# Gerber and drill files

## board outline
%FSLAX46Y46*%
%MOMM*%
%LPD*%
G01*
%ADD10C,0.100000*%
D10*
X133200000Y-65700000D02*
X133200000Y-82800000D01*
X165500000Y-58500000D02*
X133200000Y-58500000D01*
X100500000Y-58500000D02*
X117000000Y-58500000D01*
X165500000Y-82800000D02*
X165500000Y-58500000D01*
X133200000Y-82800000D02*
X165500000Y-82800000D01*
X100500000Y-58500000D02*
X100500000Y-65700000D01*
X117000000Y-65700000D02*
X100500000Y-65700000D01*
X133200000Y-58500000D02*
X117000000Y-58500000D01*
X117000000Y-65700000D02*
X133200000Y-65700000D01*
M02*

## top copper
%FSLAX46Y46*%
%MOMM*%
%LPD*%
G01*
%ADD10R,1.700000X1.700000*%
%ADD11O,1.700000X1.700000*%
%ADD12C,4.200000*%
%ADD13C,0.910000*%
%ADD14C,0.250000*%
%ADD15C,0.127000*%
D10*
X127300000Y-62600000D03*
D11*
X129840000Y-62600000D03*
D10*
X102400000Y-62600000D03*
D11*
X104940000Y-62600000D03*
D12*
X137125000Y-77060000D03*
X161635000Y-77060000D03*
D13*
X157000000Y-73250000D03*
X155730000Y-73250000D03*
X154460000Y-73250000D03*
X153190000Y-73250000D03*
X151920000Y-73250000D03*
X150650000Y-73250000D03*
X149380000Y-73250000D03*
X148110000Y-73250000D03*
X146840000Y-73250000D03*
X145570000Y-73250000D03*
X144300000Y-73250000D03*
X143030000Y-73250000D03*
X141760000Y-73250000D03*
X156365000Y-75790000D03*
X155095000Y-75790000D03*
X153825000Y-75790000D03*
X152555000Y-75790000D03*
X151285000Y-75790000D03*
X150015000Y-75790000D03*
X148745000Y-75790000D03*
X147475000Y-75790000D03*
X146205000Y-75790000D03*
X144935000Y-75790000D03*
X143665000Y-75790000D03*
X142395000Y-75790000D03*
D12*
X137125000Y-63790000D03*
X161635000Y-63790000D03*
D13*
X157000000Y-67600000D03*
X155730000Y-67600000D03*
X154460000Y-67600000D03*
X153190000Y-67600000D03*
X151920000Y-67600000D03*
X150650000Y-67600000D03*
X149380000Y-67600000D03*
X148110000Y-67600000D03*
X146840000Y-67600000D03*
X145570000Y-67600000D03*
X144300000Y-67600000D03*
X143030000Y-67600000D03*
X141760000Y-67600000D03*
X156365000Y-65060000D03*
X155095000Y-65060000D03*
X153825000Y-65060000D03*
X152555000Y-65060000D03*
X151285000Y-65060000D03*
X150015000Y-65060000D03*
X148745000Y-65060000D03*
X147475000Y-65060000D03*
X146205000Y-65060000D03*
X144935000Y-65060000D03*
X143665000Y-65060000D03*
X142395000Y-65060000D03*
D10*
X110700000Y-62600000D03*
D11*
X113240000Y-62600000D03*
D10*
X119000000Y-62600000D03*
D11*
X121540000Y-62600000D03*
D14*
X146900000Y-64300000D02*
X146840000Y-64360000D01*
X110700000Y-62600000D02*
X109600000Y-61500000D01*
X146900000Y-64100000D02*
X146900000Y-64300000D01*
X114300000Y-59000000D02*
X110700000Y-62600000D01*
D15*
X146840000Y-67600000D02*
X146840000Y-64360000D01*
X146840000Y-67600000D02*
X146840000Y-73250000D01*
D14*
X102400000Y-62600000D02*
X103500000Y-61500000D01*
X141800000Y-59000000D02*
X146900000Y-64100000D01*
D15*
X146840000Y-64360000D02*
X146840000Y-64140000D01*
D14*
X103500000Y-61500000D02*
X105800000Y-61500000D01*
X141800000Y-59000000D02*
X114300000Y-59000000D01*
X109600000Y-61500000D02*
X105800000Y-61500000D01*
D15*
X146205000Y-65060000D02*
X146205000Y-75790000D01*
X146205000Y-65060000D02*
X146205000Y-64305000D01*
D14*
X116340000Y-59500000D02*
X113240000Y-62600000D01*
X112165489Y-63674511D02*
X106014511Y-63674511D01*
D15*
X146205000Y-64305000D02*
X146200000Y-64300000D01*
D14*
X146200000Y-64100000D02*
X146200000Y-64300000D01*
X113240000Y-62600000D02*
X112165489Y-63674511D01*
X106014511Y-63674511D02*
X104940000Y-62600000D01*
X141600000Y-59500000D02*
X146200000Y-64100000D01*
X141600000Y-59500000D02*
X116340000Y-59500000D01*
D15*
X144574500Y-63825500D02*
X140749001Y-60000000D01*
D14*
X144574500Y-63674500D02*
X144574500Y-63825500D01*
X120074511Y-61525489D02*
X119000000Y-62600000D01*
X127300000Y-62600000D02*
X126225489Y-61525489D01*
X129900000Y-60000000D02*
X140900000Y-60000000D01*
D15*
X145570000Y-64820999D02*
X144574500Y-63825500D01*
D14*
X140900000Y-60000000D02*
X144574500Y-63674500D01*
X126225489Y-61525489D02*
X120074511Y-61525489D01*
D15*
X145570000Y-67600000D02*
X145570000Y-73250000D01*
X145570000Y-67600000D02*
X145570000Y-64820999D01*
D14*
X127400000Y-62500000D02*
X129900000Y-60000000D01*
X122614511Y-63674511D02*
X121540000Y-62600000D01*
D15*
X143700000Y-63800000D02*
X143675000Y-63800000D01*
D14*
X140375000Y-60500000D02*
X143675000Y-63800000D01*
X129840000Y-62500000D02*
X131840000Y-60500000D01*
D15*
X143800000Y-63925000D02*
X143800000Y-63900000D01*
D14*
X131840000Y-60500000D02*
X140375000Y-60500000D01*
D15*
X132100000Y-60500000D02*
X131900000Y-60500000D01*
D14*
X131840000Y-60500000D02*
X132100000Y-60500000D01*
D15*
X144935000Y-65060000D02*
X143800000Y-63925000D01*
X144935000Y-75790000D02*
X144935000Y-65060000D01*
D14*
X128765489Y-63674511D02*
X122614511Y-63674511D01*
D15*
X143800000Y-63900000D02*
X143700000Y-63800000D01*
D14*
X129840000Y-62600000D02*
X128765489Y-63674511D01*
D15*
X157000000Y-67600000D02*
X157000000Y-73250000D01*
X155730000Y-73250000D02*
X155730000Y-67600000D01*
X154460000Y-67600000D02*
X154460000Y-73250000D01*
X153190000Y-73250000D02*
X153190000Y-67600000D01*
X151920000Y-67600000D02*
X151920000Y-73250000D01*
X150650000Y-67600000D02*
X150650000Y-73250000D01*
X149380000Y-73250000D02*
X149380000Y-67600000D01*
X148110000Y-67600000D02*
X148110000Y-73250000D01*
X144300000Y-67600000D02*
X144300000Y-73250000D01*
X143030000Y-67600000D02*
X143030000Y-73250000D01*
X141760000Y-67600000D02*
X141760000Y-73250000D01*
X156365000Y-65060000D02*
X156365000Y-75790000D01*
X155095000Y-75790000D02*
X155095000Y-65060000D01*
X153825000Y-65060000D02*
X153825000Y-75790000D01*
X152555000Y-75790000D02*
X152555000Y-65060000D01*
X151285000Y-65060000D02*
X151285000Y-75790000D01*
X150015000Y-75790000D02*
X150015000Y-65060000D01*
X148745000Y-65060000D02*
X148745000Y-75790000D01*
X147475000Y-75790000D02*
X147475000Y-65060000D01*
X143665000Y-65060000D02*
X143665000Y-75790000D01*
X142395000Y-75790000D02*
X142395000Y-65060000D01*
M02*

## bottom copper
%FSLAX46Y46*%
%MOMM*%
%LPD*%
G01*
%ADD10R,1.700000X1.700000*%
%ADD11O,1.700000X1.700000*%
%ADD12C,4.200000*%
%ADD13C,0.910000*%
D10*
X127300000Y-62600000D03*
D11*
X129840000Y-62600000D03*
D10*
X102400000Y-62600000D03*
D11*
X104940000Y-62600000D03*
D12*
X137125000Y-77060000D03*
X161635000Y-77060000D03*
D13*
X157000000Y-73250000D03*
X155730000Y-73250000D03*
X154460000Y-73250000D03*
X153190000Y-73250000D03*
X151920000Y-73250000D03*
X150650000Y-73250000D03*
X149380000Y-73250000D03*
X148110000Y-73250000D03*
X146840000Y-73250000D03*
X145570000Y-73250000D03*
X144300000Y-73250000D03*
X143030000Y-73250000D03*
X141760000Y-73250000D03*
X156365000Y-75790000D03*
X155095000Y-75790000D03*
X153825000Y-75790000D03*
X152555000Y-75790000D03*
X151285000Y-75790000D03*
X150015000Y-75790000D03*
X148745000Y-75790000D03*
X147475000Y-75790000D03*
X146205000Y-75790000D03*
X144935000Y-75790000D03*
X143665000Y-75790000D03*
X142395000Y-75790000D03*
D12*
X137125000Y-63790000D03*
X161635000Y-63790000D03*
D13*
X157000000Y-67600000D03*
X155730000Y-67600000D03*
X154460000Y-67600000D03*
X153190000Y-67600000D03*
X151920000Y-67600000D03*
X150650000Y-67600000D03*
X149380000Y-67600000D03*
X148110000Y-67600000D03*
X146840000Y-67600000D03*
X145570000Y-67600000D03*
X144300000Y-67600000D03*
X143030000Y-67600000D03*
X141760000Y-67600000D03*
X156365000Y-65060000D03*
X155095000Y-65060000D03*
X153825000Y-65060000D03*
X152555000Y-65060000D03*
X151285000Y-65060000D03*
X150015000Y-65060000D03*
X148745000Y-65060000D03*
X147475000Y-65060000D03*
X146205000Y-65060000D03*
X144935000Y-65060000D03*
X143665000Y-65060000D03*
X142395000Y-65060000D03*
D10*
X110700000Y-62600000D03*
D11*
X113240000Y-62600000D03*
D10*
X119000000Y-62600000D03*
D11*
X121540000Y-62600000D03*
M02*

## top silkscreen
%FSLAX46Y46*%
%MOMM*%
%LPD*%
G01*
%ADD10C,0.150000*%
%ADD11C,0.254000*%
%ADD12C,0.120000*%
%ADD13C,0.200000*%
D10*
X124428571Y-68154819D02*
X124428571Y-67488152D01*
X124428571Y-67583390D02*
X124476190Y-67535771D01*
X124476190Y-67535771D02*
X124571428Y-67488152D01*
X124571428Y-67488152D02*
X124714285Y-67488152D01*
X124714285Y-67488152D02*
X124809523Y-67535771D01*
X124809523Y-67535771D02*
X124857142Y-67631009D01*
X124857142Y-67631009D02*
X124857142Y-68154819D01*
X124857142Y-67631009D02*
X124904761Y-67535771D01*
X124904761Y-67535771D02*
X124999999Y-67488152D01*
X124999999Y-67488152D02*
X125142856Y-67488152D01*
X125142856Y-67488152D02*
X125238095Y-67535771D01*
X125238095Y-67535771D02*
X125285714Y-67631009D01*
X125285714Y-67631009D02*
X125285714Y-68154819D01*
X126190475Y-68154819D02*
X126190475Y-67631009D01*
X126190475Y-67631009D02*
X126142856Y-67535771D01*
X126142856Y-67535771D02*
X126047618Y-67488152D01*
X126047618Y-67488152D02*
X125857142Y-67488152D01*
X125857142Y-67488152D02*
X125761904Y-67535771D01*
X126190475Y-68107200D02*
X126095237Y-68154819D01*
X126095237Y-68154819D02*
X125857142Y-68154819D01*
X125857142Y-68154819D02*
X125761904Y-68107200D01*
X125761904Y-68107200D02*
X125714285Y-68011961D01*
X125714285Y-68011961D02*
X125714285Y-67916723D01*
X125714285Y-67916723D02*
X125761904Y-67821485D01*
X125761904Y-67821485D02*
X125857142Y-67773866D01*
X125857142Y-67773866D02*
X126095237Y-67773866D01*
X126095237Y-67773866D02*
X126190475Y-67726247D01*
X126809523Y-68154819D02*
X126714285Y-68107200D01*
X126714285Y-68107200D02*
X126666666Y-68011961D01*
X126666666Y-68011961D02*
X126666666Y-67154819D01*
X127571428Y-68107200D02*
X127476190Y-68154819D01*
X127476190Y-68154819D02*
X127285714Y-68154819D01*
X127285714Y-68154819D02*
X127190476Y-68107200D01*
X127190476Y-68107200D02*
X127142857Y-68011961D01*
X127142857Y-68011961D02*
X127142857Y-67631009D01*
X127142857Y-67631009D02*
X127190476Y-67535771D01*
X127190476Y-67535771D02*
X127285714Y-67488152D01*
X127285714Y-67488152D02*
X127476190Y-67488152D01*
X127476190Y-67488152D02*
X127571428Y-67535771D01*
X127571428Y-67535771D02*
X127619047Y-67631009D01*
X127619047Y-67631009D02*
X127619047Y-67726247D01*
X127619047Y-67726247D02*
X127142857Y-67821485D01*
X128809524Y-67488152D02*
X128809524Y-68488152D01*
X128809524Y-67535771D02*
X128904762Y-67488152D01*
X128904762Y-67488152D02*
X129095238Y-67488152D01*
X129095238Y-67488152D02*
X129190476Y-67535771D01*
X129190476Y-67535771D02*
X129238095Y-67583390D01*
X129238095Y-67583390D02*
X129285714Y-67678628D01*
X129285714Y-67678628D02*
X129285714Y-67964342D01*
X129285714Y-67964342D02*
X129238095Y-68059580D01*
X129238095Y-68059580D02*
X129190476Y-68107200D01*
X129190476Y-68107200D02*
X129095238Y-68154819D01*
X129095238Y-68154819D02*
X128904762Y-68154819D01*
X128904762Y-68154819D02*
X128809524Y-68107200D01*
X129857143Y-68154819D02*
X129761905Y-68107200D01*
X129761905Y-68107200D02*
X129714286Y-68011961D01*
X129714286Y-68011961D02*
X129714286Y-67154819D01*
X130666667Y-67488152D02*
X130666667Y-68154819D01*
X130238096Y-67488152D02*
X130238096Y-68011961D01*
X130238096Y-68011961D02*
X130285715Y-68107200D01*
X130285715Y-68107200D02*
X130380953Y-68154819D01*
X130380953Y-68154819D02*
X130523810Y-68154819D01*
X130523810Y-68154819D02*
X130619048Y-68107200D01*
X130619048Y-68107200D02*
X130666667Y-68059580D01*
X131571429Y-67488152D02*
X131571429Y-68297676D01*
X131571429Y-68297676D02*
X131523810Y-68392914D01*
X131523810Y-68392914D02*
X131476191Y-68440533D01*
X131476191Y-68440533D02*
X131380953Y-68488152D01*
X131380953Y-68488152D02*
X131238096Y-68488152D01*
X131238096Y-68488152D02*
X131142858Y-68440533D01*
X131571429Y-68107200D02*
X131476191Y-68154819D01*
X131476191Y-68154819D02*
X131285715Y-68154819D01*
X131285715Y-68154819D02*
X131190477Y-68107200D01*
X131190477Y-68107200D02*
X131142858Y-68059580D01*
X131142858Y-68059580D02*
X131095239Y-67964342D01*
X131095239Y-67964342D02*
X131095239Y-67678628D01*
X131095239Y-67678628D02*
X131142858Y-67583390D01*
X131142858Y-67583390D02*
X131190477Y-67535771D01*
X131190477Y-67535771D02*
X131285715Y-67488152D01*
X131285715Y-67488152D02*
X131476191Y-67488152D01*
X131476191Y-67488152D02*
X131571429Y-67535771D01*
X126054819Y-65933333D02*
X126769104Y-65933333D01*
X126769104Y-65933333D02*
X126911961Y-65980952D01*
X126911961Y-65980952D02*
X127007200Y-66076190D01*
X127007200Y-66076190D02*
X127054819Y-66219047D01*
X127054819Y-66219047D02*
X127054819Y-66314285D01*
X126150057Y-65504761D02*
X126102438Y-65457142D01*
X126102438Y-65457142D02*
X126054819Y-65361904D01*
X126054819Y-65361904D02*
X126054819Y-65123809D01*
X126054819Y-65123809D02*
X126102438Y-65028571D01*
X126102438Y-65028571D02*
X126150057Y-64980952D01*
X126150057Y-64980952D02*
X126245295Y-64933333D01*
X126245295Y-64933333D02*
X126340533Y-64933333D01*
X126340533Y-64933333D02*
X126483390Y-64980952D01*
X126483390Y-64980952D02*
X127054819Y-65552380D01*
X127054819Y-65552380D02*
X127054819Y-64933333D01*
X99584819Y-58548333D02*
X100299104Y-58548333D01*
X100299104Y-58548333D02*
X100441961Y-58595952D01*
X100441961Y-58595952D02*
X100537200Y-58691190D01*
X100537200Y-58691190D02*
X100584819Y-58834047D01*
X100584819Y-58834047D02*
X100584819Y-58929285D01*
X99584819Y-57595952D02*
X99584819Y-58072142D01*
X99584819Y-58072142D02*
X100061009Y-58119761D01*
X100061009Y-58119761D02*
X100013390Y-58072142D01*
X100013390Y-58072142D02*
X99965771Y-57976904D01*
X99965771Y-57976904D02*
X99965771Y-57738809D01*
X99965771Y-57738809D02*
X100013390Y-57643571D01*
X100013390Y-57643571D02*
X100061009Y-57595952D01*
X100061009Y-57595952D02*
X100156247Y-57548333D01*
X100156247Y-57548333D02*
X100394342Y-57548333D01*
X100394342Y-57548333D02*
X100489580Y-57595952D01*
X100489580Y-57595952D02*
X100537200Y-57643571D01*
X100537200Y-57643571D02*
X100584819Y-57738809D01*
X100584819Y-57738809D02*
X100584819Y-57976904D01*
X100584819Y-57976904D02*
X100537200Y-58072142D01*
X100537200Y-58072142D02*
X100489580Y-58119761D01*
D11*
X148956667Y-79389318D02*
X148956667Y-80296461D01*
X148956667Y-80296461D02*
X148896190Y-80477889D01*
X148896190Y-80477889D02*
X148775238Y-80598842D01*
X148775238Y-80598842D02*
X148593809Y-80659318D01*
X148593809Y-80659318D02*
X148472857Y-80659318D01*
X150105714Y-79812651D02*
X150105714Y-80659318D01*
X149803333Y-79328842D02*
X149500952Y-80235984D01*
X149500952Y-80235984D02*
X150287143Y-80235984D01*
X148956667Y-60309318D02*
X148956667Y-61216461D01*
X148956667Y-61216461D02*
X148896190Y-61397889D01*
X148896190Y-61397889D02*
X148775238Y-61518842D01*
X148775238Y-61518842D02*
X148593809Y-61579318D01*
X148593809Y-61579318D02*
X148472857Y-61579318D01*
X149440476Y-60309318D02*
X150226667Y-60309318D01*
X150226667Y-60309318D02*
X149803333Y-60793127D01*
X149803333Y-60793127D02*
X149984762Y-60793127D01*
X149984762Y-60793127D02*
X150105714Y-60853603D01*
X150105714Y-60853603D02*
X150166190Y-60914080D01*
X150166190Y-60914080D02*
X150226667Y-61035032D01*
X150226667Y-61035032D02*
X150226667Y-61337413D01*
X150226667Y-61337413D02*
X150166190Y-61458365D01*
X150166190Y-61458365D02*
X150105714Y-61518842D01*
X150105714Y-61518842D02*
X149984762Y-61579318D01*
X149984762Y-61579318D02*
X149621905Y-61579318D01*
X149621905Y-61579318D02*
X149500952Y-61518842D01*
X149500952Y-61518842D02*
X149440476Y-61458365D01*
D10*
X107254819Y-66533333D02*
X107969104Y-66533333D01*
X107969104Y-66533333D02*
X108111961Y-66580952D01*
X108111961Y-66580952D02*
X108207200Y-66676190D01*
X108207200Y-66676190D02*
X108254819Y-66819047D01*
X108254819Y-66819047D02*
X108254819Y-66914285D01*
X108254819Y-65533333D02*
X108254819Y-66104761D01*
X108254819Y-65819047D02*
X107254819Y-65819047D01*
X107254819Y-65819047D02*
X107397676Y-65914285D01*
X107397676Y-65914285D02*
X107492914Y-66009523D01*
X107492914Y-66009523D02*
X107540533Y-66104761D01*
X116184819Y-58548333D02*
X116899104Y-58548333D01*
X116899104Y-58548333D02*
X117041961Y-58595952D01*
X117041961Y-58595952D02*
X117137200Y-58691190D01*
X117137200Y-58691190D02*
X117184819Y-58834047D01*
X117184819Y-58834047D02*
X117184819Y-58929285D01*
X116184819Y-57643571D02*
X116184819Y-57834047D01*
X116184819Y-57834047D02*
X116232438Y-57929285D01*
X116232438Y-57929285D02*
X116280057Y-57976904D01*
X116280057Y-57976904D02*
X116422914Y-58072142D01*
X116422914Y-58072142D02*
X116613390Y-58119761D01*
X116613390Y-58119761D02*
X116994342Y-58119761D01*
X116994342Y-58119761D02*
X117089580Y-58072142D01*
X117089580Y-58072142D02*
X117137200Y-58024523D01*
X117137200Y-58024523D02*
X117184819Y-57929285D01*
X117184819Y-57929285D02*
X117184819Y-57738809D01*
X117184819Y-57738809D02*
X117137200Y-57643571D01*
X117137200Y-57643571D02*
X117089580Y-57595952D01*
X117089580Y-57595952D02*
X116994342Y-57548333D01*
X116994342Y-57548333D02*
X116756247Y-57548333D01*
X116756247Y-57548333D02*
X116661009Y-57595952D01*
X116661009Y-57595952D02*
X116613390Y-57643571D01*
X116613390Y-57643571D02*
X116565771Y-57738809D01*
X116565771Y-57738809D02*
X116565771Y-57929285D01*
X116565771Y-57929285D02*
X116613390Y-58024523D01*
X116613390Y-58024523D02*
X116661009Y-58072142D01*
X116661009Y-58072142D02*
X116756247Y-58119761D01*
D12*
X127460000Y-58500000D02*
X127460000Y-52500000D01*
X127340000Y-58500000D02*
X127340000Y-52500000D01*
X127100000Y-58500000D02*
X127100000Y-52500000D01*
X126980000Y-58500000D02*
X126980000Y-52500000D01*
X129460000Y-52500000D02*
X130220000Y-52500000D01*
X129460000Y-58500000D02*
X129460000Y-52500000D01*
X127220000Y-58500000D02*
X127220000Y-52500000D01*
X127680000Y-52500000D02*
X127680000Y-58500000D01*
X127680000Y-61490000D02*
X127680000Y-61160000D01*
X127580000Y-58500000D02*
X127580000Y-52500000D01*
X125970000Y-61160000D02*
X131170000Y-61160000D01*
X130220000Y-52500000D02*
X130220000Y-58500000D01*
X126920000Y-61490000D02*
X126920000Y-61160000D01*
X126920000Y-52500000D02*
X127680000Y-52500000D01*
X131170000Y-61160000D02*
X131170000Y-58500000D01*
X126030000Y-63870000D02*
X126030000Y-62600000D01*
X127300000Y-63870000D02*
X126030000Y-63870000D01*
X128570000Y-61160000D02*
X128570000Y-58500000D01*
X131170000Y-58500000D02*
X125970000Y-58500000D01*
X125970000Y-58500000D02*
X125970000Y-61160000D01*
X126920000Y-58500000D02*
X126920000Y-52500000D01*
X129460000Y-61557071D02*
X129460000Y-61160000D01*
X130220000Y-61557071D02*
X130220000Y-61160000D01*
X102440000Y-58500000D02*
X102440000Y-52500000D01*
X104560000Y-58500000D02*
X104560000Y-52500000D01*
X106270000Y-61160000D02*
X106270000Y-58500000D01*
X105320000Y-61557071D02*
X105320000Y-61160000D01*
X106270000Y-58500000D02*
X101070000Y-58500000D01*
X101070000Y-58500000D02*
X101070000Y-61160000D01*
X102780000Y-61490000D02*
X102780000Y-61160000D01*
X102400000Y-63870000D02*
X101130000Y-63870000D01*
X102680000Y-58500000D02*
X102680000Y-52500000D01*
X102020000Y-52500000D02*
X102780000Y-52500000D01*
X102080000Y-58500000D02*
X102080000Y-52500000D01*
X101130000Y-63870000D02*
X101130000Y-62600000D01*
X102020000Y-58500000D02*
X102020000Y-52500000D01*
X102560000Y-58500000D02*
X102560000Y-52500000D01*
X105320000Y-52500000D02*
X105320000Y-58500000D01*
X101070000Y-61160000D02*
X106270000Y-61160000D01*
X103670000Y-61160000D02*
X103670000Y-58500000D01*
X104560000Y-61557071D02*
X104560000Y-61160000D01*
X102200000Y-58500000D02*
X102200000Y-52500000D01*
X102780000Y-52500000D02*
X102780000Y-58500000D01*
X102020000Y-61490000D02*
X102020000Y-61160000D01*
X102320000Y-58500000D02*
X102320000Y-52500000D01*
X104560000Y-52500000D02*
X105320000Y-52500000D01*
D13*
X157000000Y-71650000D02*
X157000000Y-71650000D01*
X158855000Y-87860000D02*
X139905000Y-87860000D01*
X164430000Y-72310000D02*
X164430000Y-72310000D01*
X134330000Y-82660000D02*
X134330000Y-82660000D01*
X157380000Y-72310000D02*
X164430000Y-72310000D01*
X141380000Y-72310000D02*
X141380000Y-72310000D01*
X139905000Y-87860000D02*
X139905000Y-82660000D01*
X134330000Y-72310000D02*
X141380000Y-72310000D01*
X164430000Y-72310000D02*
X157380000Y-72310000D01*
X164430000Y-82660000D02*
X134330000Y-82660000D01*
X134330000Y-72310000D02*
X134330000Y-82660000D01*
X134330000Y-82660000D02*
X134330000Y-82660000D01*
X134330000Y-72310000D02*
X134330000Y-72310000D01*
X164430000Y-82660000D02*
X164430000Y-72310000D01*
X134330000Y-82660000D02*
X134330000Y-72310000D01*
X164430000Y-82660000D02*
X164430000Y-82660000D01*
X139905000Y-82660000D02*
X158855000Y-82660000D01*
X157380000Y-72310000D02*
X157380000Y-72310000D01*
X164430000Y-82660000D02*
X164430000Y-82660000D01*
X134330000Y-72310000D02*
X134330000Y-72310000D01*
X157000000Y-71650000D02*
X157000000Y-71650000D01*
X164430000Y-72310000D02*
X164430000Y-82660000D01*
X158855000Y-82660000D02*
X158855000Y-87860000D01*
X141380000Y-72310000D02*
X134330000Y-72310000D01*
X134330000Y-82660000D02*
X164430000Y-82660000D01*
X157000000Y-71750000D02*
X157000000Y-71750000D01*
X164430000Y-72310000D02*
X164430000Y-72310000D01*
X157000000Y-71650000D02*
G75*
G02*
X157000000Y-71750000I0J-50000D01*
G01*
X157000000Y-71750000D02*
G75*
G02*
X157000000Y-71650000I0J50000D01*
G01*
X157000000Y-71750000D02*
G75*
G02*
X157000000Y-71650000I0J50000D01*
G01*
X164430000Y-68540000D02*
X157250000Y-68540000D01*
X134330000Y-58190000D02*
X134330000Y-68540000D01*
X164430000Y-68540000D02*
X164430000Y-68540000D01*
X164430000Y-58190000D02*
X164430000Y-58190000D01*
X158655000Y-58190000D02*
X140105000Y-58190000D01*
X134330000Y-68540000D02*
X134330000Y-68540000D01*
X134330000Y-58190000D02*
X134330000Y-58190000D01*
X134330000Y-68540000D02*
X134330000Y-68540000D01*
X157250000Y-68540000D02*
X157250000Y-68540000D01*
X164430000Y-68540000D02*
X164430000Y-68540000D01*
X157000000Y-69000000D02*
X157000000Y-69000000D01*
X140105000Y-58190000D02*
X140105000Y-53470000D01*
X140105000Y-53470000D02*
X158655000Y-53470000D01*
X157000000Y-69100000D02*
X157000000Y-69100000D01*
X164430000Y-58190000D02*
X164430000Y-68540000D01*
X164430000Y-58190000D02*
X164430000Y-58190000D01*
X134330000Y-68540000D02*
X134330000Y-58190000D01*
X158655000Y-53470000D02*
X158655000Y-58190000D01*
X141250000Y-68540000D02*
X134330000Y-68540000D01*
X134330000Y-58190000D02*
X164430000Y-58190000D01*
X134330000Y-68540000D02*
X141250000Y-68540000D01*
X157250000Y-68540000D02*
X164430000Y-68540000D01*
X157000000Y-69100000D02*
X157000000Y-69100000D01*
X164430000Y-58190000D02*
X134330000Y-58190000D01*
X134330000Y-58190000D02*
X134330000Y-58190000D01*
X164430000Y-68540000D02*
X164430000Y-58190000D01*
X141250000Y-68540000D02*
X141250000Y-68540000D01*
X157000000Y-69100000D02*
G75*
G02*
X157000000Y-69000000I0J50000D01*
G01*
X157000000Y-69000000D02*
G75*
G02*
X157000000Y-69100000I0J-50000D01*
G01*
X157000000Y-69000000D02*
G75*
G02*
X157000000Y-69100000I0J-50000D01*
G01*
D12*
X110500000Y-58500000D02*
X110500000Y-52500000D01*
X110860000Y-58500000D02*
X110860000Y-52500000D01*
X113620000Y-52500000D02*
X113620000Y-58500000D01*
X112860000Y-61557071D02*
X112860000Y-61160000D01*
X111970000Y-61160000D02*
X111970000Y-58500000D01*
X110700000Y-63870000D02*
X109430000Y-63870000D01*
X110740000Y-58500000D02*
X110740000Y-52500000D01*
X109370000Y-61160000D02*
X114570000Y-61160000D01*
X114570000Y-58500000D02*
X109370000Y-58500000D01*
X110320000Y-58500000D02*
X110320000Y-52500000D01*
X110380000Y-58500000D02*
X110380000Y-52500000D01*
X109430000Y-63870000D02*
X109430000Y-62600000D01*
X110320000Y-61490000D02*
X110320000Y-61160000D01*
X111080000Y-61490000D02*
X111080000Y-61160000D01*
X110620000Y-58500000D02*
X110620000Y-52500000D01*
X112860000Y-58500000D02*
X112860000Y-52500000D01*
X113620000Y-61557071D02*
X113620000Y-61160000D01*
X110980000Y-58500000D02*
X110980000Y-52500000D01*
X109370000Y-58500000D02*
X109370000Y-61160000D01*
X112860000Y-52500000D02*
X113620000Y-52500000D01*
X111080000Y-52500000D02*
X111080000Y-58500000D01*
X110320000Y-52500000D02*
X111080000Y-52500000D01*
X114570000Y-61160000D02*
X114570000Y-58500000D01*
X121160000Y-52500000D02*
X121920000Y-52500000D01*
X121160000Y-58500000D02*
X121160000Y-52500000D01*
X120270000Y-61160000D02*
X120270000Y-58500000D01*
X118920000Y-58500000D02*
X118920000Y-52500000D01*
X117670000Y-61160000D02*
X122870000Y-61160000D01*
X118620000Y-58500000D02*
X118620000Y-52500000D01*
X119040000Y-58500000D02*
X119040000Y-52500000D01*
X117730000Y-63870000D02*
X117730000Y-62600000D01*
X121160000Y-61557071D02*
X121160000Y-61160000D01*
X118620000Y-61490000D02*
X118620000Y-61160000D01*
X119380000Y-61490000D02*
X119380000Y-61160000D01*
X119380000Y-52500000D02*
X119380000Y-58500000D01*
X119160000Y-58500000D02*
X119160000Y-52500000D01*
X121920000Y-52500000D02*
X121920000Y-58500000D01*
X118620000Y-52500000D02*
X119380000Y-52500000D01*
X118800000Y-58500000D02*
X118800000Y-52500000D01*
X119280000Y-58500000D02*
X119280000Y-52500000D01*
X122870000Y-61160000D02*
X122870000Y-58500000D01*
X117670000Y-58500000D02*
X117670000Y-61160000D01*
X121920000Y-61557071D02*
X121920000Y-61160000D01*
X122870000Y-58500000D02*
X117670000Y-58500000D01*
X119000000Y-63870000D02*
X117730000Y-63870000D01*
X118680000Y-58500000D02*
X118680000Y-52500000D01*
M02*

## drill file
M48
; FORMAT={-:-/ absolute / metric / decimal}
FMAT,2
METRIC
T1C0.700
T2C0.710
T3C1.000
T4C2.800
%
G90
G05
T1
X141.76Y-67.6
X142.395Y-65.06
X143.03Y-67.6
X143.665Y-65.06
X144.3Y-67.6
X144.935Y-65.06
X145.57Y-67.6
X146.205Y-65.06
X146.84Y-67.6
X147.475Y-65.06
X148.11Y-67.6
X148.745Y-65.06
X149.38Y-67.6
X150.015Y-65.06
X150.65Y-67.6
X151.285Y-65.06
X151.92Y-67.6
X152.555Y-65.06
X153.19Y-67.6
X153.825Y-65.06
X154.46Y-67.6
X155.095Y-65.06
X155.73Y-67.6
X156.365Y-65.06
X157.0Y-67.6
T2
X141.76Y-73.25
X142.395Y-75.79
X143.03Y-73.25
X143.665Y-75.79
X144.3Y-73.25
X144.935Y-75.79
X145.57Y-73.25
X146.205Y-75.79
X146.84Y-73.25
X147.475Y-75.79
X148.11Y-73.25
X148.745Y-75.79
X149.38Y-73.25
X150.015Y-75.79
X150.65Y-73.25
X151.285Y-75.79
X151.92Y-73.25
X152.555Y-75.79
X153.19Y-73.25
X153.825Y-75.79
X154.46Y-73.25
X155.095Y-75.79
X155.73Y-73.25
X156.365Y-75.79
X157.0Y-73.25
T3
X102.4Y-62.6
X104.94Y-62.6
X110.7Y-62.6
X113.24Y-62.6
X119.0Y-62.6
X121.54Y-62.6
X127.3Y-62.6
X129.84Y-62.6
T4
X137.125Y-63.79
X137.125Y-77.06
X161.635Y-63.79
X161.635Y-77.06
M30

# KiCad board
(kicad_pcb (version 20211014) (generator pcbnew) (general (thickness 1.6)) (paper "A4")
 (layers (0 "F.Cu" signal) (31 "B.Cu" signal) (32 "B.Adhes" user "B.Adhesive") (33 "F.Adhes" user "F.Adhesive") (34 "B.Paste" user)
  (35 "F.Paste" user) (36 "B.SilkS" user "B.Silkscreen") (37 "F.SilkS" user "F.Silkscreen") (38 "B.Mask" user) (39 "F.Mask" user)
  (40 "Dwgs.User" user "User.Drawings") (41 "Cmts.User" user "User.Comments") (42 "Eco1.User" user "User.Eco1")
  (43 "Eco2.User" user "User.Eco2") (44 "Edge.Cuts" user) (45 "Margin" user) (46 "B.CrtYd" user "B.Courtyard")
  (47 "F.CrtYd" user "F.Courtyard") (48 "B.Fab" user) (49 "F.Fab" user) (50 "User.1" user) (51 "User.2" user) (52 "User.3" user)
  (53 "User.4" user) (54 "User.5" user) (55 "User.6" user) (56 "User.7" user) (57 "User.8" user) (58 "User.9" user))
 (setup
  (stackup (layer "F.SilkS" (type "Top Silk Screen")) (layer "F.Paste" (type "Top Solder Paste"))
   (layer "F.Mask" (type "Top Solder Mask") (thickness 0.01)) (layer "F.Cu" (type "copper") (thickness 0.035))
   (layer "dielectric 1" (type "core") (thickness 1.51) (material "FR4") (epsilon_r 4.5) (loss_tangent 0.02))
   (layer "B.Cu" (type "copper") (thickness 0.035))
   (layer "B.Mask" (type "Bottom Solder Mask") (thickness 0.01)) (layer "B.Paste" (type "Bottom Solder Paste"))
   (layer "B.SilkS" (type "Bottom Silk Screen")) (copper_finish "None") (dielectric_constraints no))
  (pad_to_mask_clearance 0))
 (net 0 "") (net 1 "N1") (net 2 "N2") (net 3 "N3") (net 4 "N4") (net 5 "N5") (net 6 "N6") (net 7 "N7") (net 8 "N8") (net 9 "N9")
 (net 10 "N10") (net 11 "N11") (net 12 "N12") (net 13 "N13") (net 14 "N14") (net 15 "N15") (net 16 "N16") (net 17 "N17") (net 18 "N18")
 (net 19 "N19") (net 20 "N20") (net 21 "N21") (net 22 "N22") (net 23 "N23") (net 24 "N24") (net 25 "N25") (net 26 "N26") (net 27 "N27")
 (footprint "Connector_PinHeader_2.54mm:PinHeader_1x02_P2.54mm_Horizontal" (layer "F.Cu") (at 127.3 62.6 90)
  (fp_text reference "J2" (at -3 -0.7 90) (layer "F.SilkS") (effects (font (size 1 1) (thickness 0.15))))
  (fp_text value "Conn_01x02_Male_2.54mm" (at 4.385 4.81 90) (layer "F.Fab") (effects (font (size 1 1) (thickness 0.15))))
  (fp_line (start 4.1 0.16) (end 10.1 0.16) (layer "F.SilkS") (width 0.12))
  (fp_line (start 4.1 0.04) (end 10.1 0.04) (layer "F.SilkS") (width 0.12))
  (fp_line (start 4.1 -0.2) (end 10.1 -0.2) (layer "F.SilkS") (width 0.12))
  (fp_line (start 4.1 -0.32) (end 10.1 -0.32) (layer "F.SilkS") (width 0.12))
  (fp_line (start 10.1 2.16) (end 10.1 2.92) (layer "F.SilkS") (width 0.12))
  (fp_line (start 4.1 2.16) (end 10.1 2.16) (layer "F.SilkS") (width 0.12))
  (fp_line (start 4.1 -0.08) (end 10.1 -0.08) (layer "F.SilkS") (width 0.12))
  (fp_line (start 10.1 0.38) (end 4.1 0.38) (layer "F.SilkS") (width 0.12))
  (fp_line (start 1.11 0.38) (end 1.44 0.38) (layer "F.SilkS") (width 0.12))
  (fp_line (start 4.1 0.28) (end 10.1 0.28) (layer "F.SilkS") (width 0.12))
  (fp_line (start 1.44 -1.33) (end 1.44 3.87) (layer "F.SilkS") (width 0.12))
  (fp_line (start 10.1 2.92) (end 4.1 2.92) (layer "F.SilkS") (width 0.12))
  (fp_line (start 1.11 -0.38) (end 1.44 -0.38) (layer "F.SilkS") (width 0.12))
  (fp_line (start 10.1 -0.38) (end 10.1 0.38) (layer "F.SilkS") (width 0.12))
  (fp_line (start 1.44 3.87) (end 4.1 3.87) (layer "F.SilkS") (width 0.12))
  (fp_line (start -1.27 -1.27) (end 0 -1.27) (layer "F.SilkS") (width 0.12))
  (fp_line (start -1.27 0) (end -1.27 -1.27) (layer "F.SilkS") (width 0.12))
  (fp_line (start 1.44 1.27) (end 4.1 1.27) (layer "F.SilkS") (width 0.12))
  (fp_line (start 4.1 3.87) (end 4.1 -1.33) (layer "F.SilkS") (width 0.12))
  (fp_line (start 4.1 -1.33) (end 1.44 -1.33) (layer "F.SilkS") (width 0.12))
  (fp_line (start 4.1 -0.38) (end 10.1 -0.38) (layer "F.SilkS") (width 0.12))
  (fp_line (start 1.042929 2.16) (end 1.44 2.16) (layer "F.SilkS") (width 0.12))
  (fp_line (start 1.042929 2.92) (end 1.44 2.92) (layer "F.SilkS") (width 0.12))
  (pad "1" thru_hole rect (at 0 0 90) (size 1.7 1.7) (drill 1) (layers *.Cu *.Mask) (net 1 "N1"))
  (pad "2" thru_hole oval (at 0 2.54 90) (size 1.7 1.7) (drill 1) (layers *.Cu *.Mask) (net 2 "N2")))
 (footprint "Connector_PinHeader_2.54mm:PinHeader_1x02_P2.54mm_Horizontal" (layer "F.Cu") (at 102.4 62.6 90)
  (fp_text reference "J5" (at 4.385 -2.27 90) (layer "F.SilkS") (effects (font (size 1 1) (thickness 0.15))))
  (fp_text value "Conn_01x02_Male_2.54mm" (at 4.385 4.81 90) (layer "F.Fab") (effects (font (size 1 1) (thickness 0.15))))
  (fp_line (start 4.1 0.04) (end 10.1 0.04) (layer "F.SilkS") (width 0.12))
  (fp_line (start 4.1 2.16) (end 10.1 2.16) (layer "F.SilkS") (width 0.12))
  (fp_line (start 1.44 3.87) (end 4.1 3.87) (layer "F.SilkS") (width 0.12))
  (fp_line (start 1.042929 2.92) (end 1.44 2.92) (layer "F.SilkS") (width 0.12))
  (fp_line (start 4.1 3.87) (end 4.1 -1.33) (layer "F.SilkS") (width 0.12))
  (fp_line (start 4.1 -1.33) (end 1.44 -1.33) (layer "F.SilkS") (width 0.12))
  (fp_line (start 1.11 0.38) (end 1.44 0.38) (layer "F.SilkS") (width 0.12))
  (fp_line (start -1.27 0) (end -1.27 -1.27) (layer "F.SilkS") (width 0.12))
  (fp_line (start 4.1 0.28) (end 10.1 0.28) (layer "F.SilkS") (width 0.12))
  (fp_line (start 10.1 -0.38) (end 10.1 0.38) (layer "F.SilkS") (width 0.12))
  (fp_line (start 4.1 -0.32) (end 10.1 -0.32) (layer "F.SilkS") (width 0.12))
  (fp_line (start -1.27 -1.27) (end 0 -1.27) (layer "F.SilkS") (width 0.12))
  (fp_line (start 4.1 -0.38) (end 10.1 -0.38) (layer "F.SilkS") (width 0.12))
  (fp_line (start 4.1 0.16) (end 10.1 0.16) (layer "F.SilkS") (width 0.12))
  (fp_line (start 10.1 2.92) (end 4.1 2.92) (layer "F.SilkS") (width 0.12))
  (fp_line (start 1.44 -1.33) (end 1.44 3.87) (layer "F.SilkS") (width 0.12))
  (fp_line (start 1.44 1.27) (end 4.1 1.27) (layer "F.SilkS") (width 0.12))
  (fp_line (start 1.042929 2.16) (end 1.44 2.16) (layer "F.SilkS") (width 0.12))
  (fp_line (start 4.1 -0.2) (end 10.1 -0.2) (layer "F.SilkS") (width 0.12))
  (fp_line (start 10.1 0.38) (end 4.1 0.38) (layer "F.SilkS") (width 0.12))
  (fp_line (start 1.11 -0.38) (end 1.44 -0.38) (layer "F.SilkS") (width 0.12))
  (fp_line (start 4.1 -0.08) (end 10.1 -0.08) (layer "F.SilkS") (width 0.12))
  (fp_line (start 10.1 2.16) (end 10.1 2.92) (layer "F.SilkS") (width 0.12))
  (pad "1" thru_hole rect (at 0 0 90) (size 1.7 1.7) (drill 1) (layers *.Cu *.Mask) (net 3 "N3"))
  (pad "2" thru_hole oval (at 0 2.54 90) (size 1.7 1.7) (drill 1) (layers *.Cu *.Mask) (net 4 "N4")))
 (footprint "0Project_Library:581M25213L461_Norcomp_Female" (layer "F.Cu") (at 157 73.25)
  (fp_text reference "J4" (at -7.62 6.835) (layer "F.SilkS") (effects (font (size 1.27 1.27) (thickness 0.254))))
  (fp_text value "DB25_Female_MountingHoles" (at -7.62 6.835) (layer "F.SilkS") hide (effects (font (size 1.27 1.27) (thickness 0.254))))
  (fp_line (start 0 -1.6) (end 0 -1.6) (layer "F.SilkS") (width 0.2))
  (fp_line (start 1.855 14.61) (end -17.095 14.61) (layer "F.SilkS") (width 0.2))
  (fp_line (start 7.43 -0.94) (end 7.43 -0.94) (layer "F.SilkS") (width 0.2))
  (fp_line (start -22.67 9.41) (end -22.67 9.41) (layer "F.SilkS") (width 0.2))
  (fp_line (start 0.38 -0.94) (end 7.43 -0.94) (layer "F.SilkS") (width 0.2))
  (fp_line (start -15.62 -0.94) (end -15.62 -0.94) (layer "F.SilkS") (width 0.2))
  (fp_line (start -17.095 14.61) (end -17.095 9.41) (layer "F.SilkS") (width 0.2))
  (fp_line (start -22.67 -0.94) (end -15.62 -0.94) (layer "F.SilkS") (width 0.2))
  (fp_line (start 7.43 -0.94) (end 0.38 -0.94) (layer "F.SilkS") (width 0.2))
  (fp_line (start 7.43 9.41) (end -22.67 9.41) (layer "F.SilkS") (width 0.2))
  (fp_line (start -22.67 -0.94) (end -22.67 9.41) (layer "F.SilkS") (width 0.2))
  (fp_line (start -22.67 9.41) (end -22.67 9.41) (layer "F.SilkS") (width 0.2))
  (fp_line (start -22.67 -0.94) (end -22.67 -0.94) (layer "F.SilkS") (width 0.2))
  (fp_line (start 7.43 9.41) (end 7.43 -0.94) (layer "F.SilkS") (width 0.2))
  (fp_line (start -22.67 9.41) (end -22.67 -0.94) (layer "F.SilkS") (width 0.2))
  (fp_line (start 7.43 9.41) (end 7.43 9.41) (layer "F.SilkS") (width 0.2))
  (fp_line (start -17.095 9.41) (end 1.855 9.41) (layer "F.SilkS") (width 0.2))
  (fp_line (start 0.38 -0.94) (end 0.38 -0.94) (layer "F.SilkS") (width 0.2))
  (fp_line (start 7.43 9.41) (end 7.43 9.41) (layer "F.SilkS") (width 0.2))
  (fp_line (start -22.67 -0.94) (end -22.67 -0.94) (layer "F.SilkS") (width 0.2))
  (fp_line (start 0 -1.6) (end 0 -1.6) (layer "F.SilkS") (width 0.2))
  (fp_line (start 7.43 -0.94) (end 7.43 9.41) (layer "F.SilkS") (width 0.2))
  (fp_line (start 1.855 9.41) (end 1.855 14.61) (layer "F.SilkS") (width 0.2))
  (fp_line (start -15.62 -0.94) (end -22.67 -0.94) (layer "F.SilkS") (width 0.2))
  (fp_line (start -22.67 9.41) (end 7.43 9.41) (layer "F.SilkS") (width 0.2))
  (fp_line (start 0 -1.5) (end 0 -1.5) (layer "F.SilkS") (width 0.2))
  (fp_line (start 7.43 -0.94) (end 7.43 -0.94) (layer "F.SilkS") (width 0.2))
  (fp_arc (start 0 -1.6) (mid 0.05 -1.55) (end 0 -1.5) (layer "F.SilkS") (width 0.2))
  (fp_arc (start 0 -1.5) (mid -0.05 -1.55) (end 0 -1.6) (layer "F.SilkS") (width 0.2))
  (fp_arc (start 0 -1.5) (mid -0.05 -1.55) (end 0 -1.6) (layer "F.SilkS") (width 0.2))
  (pad "0" thru_hole circle (at -19.875 3.81) (size 4.2 4.2) (drill 2.8) (layers *.Cu *.Mask) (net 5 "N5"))
  (pad "0" thru_hole circle (at 4.635 3.81) (size 4.2 4.2) (drill 2.8) (layers *.Cu *.Mask) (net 5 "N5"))
  (pad "1" thru_hole circle (at 0 0) (size 0.91 0.91) (drill 0.71) (layers *.Cu *.Mask) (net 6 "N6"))
  (pad "2" thru_hole circle (at -1.27 0) (size 0.91 0.91) (drill 0.71) (layers *.Cu *.Mask) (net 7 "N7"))
  (pad "3" thru_hole circle (at -2.54 0) (size 0.91 0.91) (drill 0.71) (layers *.Cu *.Mask) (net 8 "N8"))
  (pad "4" thru_hole circle (at -3.81 0) (size 0.91 0.91) (drill 0.71) (layers *.Cu *.Mask) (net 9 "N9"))
  (pad "5" thru_hole circle (at -5.08 0) (size 0.91 0.91) (drill 0.71) (layers *.Cu *.Mask) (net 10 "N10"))
  (pad "6" thru_hole circle (at -6.35 0) (size 0.91 0.91) (drill 0.71) (layers *.Cu *.Mask) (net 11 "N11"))
  (pad "7" thru_hole circle (at -7.62 0) (size 0.91 0.91) (drill 0.71) (layers *.Cu *.Mask) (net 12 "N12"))
  (pad "8" thru_hole circle (at -8.89 0) (size 0.91 0.91) (drill 0.71) (layers *.Cu *.Mask) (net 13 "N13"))
  (pad "9" thru_hole circle (at -10.16 0) (size 0.91 0.91) (drill 0.71) (layers *.Cu *.Mask) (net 3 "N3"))
  (pad "10" thru_hole circle (at -11.43 0) (size 0.91 0.91) (drill 0.71) (layers *.Cu *.Mask) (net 1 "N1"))
  (pad "11" thru_hole circle (at -12.7 0) (size 0.91 0.91) (drill 0.71) (layers *.Cu *.Mask) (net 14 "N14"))
  (pad "12" thru_hole circle (at -13.97 0) (size 0.91 0.91) (drill 0.71) (layers *.Cu *.Mask) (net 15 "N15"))
  (pad "13" thru_hole circle (at -15.24 0) (size 0.91 0.91) (drill 0.71) (layers *.Cu *.Mask) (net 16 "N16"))
  (pad "14" thru_hole circle (at -0.635 2.54) (size 0.91 0.91) (drill 0.71) (layers *.Cu *.Mask) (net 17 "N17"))
  (pad "15" thru_hole circle (at -1.905 2.54) (size 0.91 0.91) (drill 0.71) (layers *.Cu *.Mask) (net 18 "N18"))
  (pad "16" thru_hole circle (at -3.175 2.54) (size 0.91 0.91) (drill 0.71) (layers *.Cu *.Mask) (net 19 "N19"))
  (pad "17" thru_hole circle (at -4.445 2.54) (size 0.91 0.91) (drill 0.71) (layers *.Cu *.Mask) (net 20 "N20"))
  (pad "18" thru_hole circle (at -5.715 2.54) (size 0.91 0.91) (drill 0.71) (layers *.Cu *.Mask) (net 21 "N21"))
  (pad "19" thru_hole circle (at -6.985 2.54) (size 0.91 0.91) (drill 0.71) (layers *.Cu *.Mask) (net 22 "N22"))
  (pad "20" thru_hole circle (at -8.255 2.54) (size 0.91 0.91) (drill 0.71) (layers *.Cu *.Mask) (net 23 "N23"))
  (pad "21" thru_hole circle (at -9.525 2.54) (size 0.91 0.91) (drill 0.71) (layers *.Cu *.Mask) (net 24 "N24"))
  (pad "22" thru_hole circle (at -10.795 2.54) (size 0.91 0.91) (drill 0.71) (layers *.Cu *.Mask) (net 4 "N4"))
  (pad "23" thru_hole circle (at -12.065 2.54) (size 0.91 0.91) (drill 0.71) (layers *.Cu *.Mask) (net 2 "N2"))
  (pad "24" thru_hole circle (at -13.335 2.54) (size 0.91 0.91) (drill 0.71) (layers *.Cu *.Mask) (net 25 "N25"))
  (pad "25" thru_hole circle (at -14.605 2.54) (size 0.91 0.91) (drill 0.71) (layers *.Cu *.Mask) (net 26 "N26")))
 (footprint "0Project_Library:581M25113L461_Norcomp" (layer "F.Cu") (at 157 67.6 180)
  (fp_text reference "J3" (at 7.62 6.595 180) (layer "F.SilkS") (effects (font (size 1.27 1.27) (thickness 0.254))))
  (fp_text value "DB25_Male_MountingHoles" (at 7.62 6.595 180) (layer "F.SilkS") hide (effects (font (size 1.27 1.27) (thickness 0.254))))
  (fp_line (start -7.43 -0.94) (end -0.25 -0.94) (layer "F.SilkS") (width 0.2))
  (fp_line (start 22.67 9.41) (end 22.67 -0.94) (layer "F.SilkS") (width 0.2))
  (fp_line (start -7.43 -0.94) (end -7.43 -0.94) (layer "F.SilkS") (width 0.2))
  (fp_line (start -7.43 9.41) (end -7.43 9.41) (layer "F.SilkS") (width 0.2))
  (fp_line (start -1.655 9.41) (end 16.895 9.41) (layer "F.SilkS") (width 0.2))
  (fp_line (start 22.67 -0.94) (end 22.67 -0.94) (layer "F.SilkS") (width 0.2))
  (fp_line (start 22.67 9.41) (end 22.67 9.41) (layer "F.SilkS") (width 0.2))
  (fp_line (start 22.67 -0.94) (end 22.67 -0.94) (layer "F.SilkS") (width 0.2))
  (fp_line (start -0.25 -0.94) (end -0.25 -0.94) (layer "F.SilkS") (width 0.2))
  (fp_line (start -7.43 -0.94) (end -7.43 -0.94) (layer "F.SilkS") (width 0.2))
  (fp_line (start 0 -1.4) (end 0 -1.4) (layer "F.SilkS") (width 0.2))
  (fp_line (start 16.895 9.41) (end 16.895 14.13) (layer "F.SilkS") (width 0.2))
  (fp_line (start 16.895 14.13) (end -1.655 14.13) (layer "F.SilkS") (width 0.2))
  (fp_line (start 0 -1.5) (end 0 -1.5) (layer "F.SilkS") (width 0.2))
  (fp_line (start -7.43 9.41) (end -7.43 -0.94) (layer "F.SilkS") (width 0.2))
  (fp_line (start -7.43 9.41) (end -7.43 9.41) (layer "F.SilkS") (width 0.2))
  (fp_line (start 22.67 -0.94) (end 22.67 9.41) (layer "F.SilkS") (width 0.2))
  (fp_line (start -1.655 14.13) (end -1.655 9.41) (layer "F.SilkS") (width 0.2))
  (fp_line (start 15.75 -0.94) (end 22.67 -0.94) (layer "F.SilkS") (width 0.2))
  (fp_line (start 22.67 9.41) (end -7.43 9.41) (layer "F.SilkS") (width 0.2))
  (fp_line (start 22.67 -0.94) (end 15.75 -0.94) (layer "F.SilkS") (width 0.2))
  (fp_line (start -0.25 -0.94) (end -7.43 -0.94) (layer "F.SilkS") (width 0.2))
  (fp_line (start 0 -1.5) (end 0 -1.5) (layer "F.SilkS") (width 0.2))
  (fp_line (start -7.43 9.41) (end 22.67 9.41) (layer "F.SilkS") (width 0.2))
  (fp_line (start 22.67 9.41) (end 22.67 9.41) (layer "F.SilkS") (width 0.2))
  (fp_line (start -7.43 -0.94) (end -7.43 9.41) (layer "F.SilkS") (width 0.2))
  (fp_line (start 15.75 -0.94) (end 15.75 -0.94) (layer "F.SilkS") (width 0.2))
  (fp_arc (start 0 -1.5) (mid 0.05 -1.45) (end 0 -1.4) (layer "F.SilkS") (width 0.2))
  (fp_arc (start 0 -1.4) (mid -0.05 -1.45) (end 0 -1.5) (layer "F.SilkS") (width 0.2))
  (fp_arc (start 0 -1.4) (mid -0.05 -1.45) (end 0 -1.5) (layer "F.SilkS") (width 0.2))
  (pad "0" thru_hole circle (at 19.875 3.81 180) (size 4.2 4.2) (drill 2.8) (layers *.Cu *.Mask) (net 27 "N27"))
  (pad "0" thru_hole circle (at -4.635 3.81 180) (size 4.2 4.2) (drill 2.8) (layers *.Cu *.Mask) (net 27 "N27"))
  (pad "1" thru_hole circle (at 0 0 180) (size 0.91 0.91) (drill 0.7) (layers *.Cu *.Mask) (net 6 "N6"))
  (pad "2" thru_hole circle (at 1.27 0 180) (size 0.91 0.91) (drill 0.7) (layers *.Cu *.Mask) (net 7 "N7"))
  (pad "3" thru_hole circle (at 2.54 0 180) (size 0.91 0.91) (drill 0.7) (layers *.Cu *.Mask) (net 8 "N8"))
  (pad "4" thru_hole circle (at 3.81 0 180) (size 0.91 0.91) (drill 0.7) (layers *.Cu *.Mask) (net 9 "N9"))
  (pad "5" thru_hole circle (at 5.08 0 180) (size 0.91 0.91) (drill 0.7) (layers *.Cu *.Mask) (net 10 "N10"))
  (pad "6" thru_hole circle (at 6.35 0 180) (size 0.91 0.91) (drill 0.7) (layers *.Cu *.Mask) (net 11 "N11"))
  (pad "7" thru_hole circle (at 7.62 0 180) (size 0.91 0.91) (drill 0.7) (layers *.Cu *.Mask) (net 12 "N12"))
  (pad "8" thru_hole circle (at 8.89 0 180) (size 0.91 0.91) (drill 0.7) (layers *.Cu *.Mask) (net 13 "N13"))
  (pad "9" thru_hole circle (at 10.16 0 180) (size 0.91 0.91) (drill 0.7) (layers *.Cu *.Mask) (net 3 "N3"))
  (pad "10" thru_hole circle (at 11.43 0 180) (size 0.91 0.91) (drill 0.7) (layers *.Cu *.Mask) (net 1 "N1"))
  (pad "11" thru_hole circle (at 12.7 0 180) (size 0.91 0.91) (drill 0.7) (layers *.Cu *.Mask) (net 14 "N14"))
  (pad "12" thru_hole circle (at 13.97 0 180) (size 0.91 0.91) (drill 0.7) (layers *.Cu *.Mask) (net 15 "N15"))
  (pad "13" thru_hole circle (at 15.24 0 180) (size 0.91 0.91) (drill 0.7) (layers *.Cu *.Mask) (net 16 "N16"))
  (pad "14" thru_hole circle (at 0.635 2.54 180) (size 0.91 0.91) (drill 0.7) (layers *.Cu *.Mask) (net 17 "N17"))
  (pad "15" thru_hole circle (at 1.905 2.54 180) (size 0.91 0.91) (drill 0.7) (layers *.Cu *.Mask) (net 18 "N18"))
  (pad "16" thru_hole circle (at 3.175 2.54 180) (size 0.91 0.91) (drill 0.7) (layers *.Cu *.Mask) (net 19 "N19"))
  (pad "17" thru_hole circle (at 4.445 2.54 180) (size 0.91 0.91) (drill 0.7) (layers *.Cu *.Mask) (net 20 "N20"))
  (pad "18" thru_hole circle (at 5.715 2.54 180) (size 0.91 0.91) (drill 0.7) (layers *.Cu *.Mask) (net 21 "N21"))
  (pad "19" thru_hole circle (at 6.985 2.54 180) (size 0.91 0.91) (drill 0.7) (layers *.Cu *.Mask) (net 22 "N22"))
  (pad "20" thru_hole circle (at 8.255 2.54 180) (size 0.91 0.91) (drill 0.7) (layers *.Cu *.Mask) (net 23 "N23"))
  (pad "21" thru_hole circle (at 9.525 2.54 180) (size 0.91 0.91) (drill 0.7) (layers *.Cu *.Mask) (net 24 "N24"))
  (pad "22" thru_hole circle (at 10.795 2.54 180) (size 0.91 0.91) (drill 0.7) (layers *.Cu *.Mask) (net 4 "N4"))
  (pad "23" thru_hole circle (at 12.065 2.54 180) (size 0.91 0.91) (drill 0.7) (layers *.Cu *.Mask) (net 2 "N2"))
  (pad "24" thru_hole circle (at 13.335 2.54 180) (size 0.91 0.91) (drill 0.7) (layers *.Cu *.Mask) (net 25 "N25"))
  (pad "25" thru_hole circle (at 14.605 2.54 180) (size 0.91 0.91) (drill 0.7) (layers *.Cu *.Mask) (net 26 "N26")))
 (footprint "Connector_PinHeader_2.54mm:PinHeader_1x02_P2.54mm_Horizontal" (layer "F.Cu") (at 110.7 62.6 90)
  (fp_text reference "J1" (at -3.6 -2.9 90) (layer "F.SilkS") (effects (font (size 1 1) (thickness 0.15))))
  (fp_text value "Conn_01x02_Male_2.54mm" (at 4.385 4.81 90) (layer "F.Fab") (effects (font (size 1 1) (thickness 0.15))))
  (fp_line (start 4.1 -0.2) (end 10.1 -0.2) (layer "F.SilkS") (width 0.12))
  (fp_line (start 4.1 0.16) (end 10.1 0.16) (layer "F.SilkS") (width 0.12))
  (fp_line (start 10.1 2.92) (end 4.1 2.92) (layer "F.SilkS") (width 0.12))
  (fp_line (start 1.042929 2.16) (end 1.44 2.16) (layer "F.SilkS") (width 0.12))
  (fp_line (start 1.44 1.27) (end 4.1 1.27) (layer "F.SilkS") (width 0.12))
  (fp_line (start -1.27 0) (end -1.27 -1.27) (layer "F.SilkS") (width 0.12))
  (fp_line (start 4.1 0.04) (end 10.1 0.04) (layer "F.SilkS") (width 0.12))
  (fp_line (start 1.44 -1.33) (end 1.44 3.87) (layer "F.SilkS") (width 0.12))
  (fp_line (start 4.1 3.87) (end 4.1 -1.33) (layer "F.SilkS") (width 0.12))
  (fp_line (start 4.1 -0.38) (end 10.1 -0.38) (layer "F.SilkS") (width 0.12))
  (fp_line (start 4.1 -0.32) (end 10.1 -0.32) (layer "F.SilkS") (width 0.12))
  (fp_line (start -1.27 -1.27) (end 0 -1.27) (layer "F.SilkS") (width 0.12))
  (fp_line (start 1.11 -0.38) (end 1.44 -0.38) (layer "F.SilkS") (width 0.12))
  (fp_line (start 1.11 0.38) (end 1.44 0.38) (layer "F.SilkS") (width 0.12))
  (fp_line (start 4.1 -0.08) (end 10.1 -0.08) (layer "F.SilkS") (width 0.12))
  (fp_line (start 4.1 2.16) (end 10.1 2.16) (layer "F.SilkS") (width 0.12))
  (fp_line (start 1.042929 2.92) (end 1.44 2.92) (layer "F.SilkS") (width 0.12))
  (fp_line (start 4.1 0.28) (end 10.1 0.28) (layer "F.SilkS") (width 0.12))
  (fp_line (start 4.1 -1.33) (end 1.44 -1.33) (layer "F.SilkS") (width 0.12))
  (fp_line (start 10.1 2.16) (end 10.1 2.92) (layer "F.SilkS") (width 0.12))
  (fp_line (start 10.1 0.38) (end 4.1 0.38) (layer "F.SilkS") (width 0.12))
  (fp_line (start 10.1 -0.38) (end 10.1 0.38) (layer "F.SilkS") (width 0.12))
  (fp_line (start 1.44 3.87) (end 4.1 3.87) (layer "F.SilkS") (width 0.12))
  (pad "1" thru_hole rect (at 0 0 90) (size 1.7 1.7) (drill 1) (layers *.Cu *.Mask) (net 3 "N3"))
  (pad "2" thru_hole oval (at 0 2.54 90) (size 1.7 1.7) (drill 1) (layers *.Cu *.Mask) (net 4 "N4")))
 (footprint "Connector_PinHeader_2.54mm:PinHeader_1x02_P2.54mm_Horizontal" (layer "F.Cu") (at 119 62.6 90)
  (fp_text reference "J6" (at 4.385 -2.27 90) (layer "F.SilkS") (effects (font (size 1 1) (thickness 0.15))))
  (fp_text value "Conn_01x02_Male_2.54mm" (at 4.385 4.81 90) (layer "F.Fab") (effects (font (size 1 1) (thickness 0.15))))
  (fp_line (start 10.1 2.16) (end 10.1 2.92) (layer "F.SilkS") (width 0.12))
  (fp_line (start 4.1 2.16) (end 10.1 2.16) (layer "F.SilkS") (width 0.12))
  (fp_line (start 1.44 1.27) (end 4.1 1.27) (layer "F.SilkS") (width 0.12))
  (fp_line (start 4.1 -0.08) (end 10.1 -0.08) (layer "F.SilkS") (width 0.12))
  (fp_line (start 1.44 -1.33) (end 1.44 3.87) (layer "F.SilkS") (width 0.12))
  (fp_line (start 4.1 -0.38) (end 10.1 -0.38) (layer "F.SilkS") (width 0.12))
  (fp_line (start 4.1 0.04) (end 10.1 0.04) (layer "F.SilkS") (width 0.12))
  (fp_line (start -1.27 -1.27) (end 0 -1.27) (layer "F.SilkS") (width 0.12))
  (fp_line (start 1.042929 2.16) (end 1.44 2.16) (layer "F.SilkS") (width 0.12))
  (fp_line (start 1.11 -0.38) (end 1.44 -0.38) (layer "F.SilkS") (width 0.12))
  (fp_line (start 1.11 0.38) (end 1.44 0.38) (layer "F.SilkS") (width 0.12))
  (fp_line (start 10.1 0.38) (end 4.1 0.38) (layer "F.SilkS") (width 0.12))
  (fp_line (start 4.1 0.16) (end 10.1 0.16) (layer "F.SilkS") (width 0.12))
  (fp_line (start 10.1 2.92) (end 4.1 2.92) (layer "F.SilkS") (width 0.12))
  (fp_line (start 10.1 -0.38) (end 10.1 0.38) (layer "F.SilkS") (width 0.12))
  (fp_line (start 4.1 -0.2) (end 10.1 -0.2) (layer "F.SilkS") (width 0.12))
  (fp_line (start 4.1 0.28) (end 10.1 0.28) (layer "F.SilkS") (width 0.12))
  (fp_line (start 1.44 3.87) (end 4.1 3.87) (layer "F.SilkS") (width 0.12))
  (fp_line (start 4.1 -1.33) (end 1.44 -1.33) (layer "F.SilkS") (width 0.12))
  (fp_line (start 1.042929 2.92) (end 1.44 2.92) (layer "F.SilkS") (width 0.12))
  (fp_line (start 4.1 3.87) (end 4.1 -1.33) (layer "F.SilkS") (width 0.12))
  (fp_line (start -1.27 0) (end -1.27 -1.27) (layer "F.SilkS") (width 0.12))
  (fp_line (start 4.1 -0.32) (end 10.1 -0.32) (layer "F.SilkS") (width 0.12))
  (pad "1" thru_hole rect (at 0 0 90) (size 1.7 1.7) (drill 1) (layers *.Cu *.Mask) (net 1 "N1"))
  (pad "2" thru_hole oval (at 0 2.54 90) (size 1.7 1.7) (drill 1) (layers *.Cu *.Mask) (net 2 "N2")))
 (gr_line (start 133.2 65.7) (end 133.2 82.8) (layer "Edge.Cuts") (width 0.1))
 (gr_line (start 165.5 58.5) (end 133.2 58.5) (layer "Edge.Cuts") (width 0.1))
 (gr_line (start 100.5 58.5) (end 117 58.5) (layer "Edge.Cuts") (width 0.1))
 (gr_line (start 165.5 82.8) (end 165.5 58.5) (layer "Edge.Cuts") (width 0.1))
 (gr_line (start 133.2 82.8) (end 165.5 82.8) (layer "Edge.Cuts") (width 0.1))
 (gr_line (start 100.5 58.5) (end 100.5 65.7) (layer "Edge.Cuts") (width 0.1))
 (gr_line (start 117 65.7) (end 100.5 65.7) (layer "Edge.Cuts") (width 0.1))
 (gr_line (start 133.2 58.5) (end 117 58.5) (layer "Edge.Cuts") (width 0.1))
 (gr_line (start 117 65.7) (end 133.2 65.7) (layer "Edge.Cuts") (width 0.1))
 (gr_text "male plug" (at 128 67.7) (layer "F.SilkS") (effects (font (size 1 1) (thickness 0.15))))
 (segment (start 146.9 64.3) (end 146.84 64.36) (width 0.25) (layer "F.Cu") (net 3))
 (segment (start 110.7 62.6) (end 109.6 61.5) (width 0.25) (layer "F.Cu") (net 3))
 (segment (start 146.9 64.1) (end 146.9 64.3) (width 0.25) (layer "F.Cu") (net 3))
 (segment (start 114.3 59) (end 110.7 62.6) (width 0.25) (layer "F.Cu") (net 3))
 (segment (start 146.84 67.6) (end 146.84 64.36) (width 0.127) (layer "F.Cu") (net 3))
 (segment (start 146.84 67.6) (end 146.84 73.25) (width 0.127) (layer "F.Cu") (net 3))
 (segment (start 102.4 62.6) (end 103.5 61.5) (width 0.25) (layer "F.Cu") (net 3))
 (segment (start 141.8 59) (end 146.9 64.1) (width 0.25) (layer "F.Cu") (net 3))
 (segment (start 146.84 64.36) (end 146.84 64.14) (width 0.127) (layer "F.Cu") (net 3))
 (segment (start 103.5 61.5) (end 105.8 61.5) (width 0.25) (layer "F.Cu") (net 3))
 (segment (start 141.8 59) (end 114.3 59) (width 0.25) (layer "F.Cu") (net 3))
 (segment (start 109.6 61.5) (end 105.8 61.5) (width 0.25) (layer "F.Cu") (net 3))
 (segment (start 146.205 65.06) (end 146.205 75.79) (width 0.127) (layer "F.Cu") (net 4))
 (segment (start 146.205 65.06) (end 146.205 64.305) (width 0.127) (layer "F.Cu") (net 4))
 (segment (start 116.34 59.5) (end 113.24 62.6) (width 0.25) (layer "F.Cu") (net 4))
 (segment (start 112.165489 63.674511) (end 106.014511 63.674511) (width 0.25) (layer "F.Cu") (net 4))
 (segment (start 146.205 64.305) (end 146.2 64.3) (width 0.127) (layer "F.Cu") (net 4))
 (segment (start 146.2 64.1) (end 146.2 64.3) (width 0.25) (layer "F.Cu") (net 4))
 (segment (start 113.24 62.6) (end 112.165489 63.674511) (width 0.25) (layer "F.Cu") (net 4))
 (segment (start 106.014511 63.674511) (end 104.94 62.6) (width 0.25) (layer "F.Cu") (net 4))
 (segment (start 141.6 59.5) (end 146.2 64.1) (width 0.25) (layer "F.Cu") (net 4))
 (segment (start 141.6 59.5) (end 116.34 59.5) (width 0.25) (layer "F.Cu") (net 4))
 (segment (start 144.5745 63.8255) (end 140.749001 60) (width 0.127) (layer "F.Cu") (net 1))
 (segment (start 144.5745 63.6745) (end 144.5745 63.8255) (width 0.25) (layer "F.Cu") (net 1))
 (segment (start 120.074511 61.525489) (end 119 62.6) (width 0.25) (layer "F.Cu") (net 1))
 (segment (start 127.3 62.6) (end 126.225489 61.525489) (width 0.25) (layer "F.Cu") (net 1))
 (segment (start 129.9 60) (end 140.9 60) (width 0.25) (layer "F.Cu") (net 1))
 (segment (start 145.57 64.820999) (end 144.5745 63.8255) (width 0.127) (layer "F.Cu") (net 1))
 (segment (start 140.9 60) (end 144.5745 63.6745) (width 0.25) (layer "F.Cu") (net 1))
 (segment (start 126.225489 61.525489) (end 120.074511 61.525489) (width 0.25) (layer "F.Cu") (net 1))
 (segment (start 145.57 67.6) (end 145.57 73.25) (width 0.127) (layer "F.Cu") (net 1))
 (segment (start 145.57 67.6) (end 145.57 64.820999) (width 0.127) (layer "F.Cu") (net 1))
 (segment (start 127.4 62.5) (end 129.9 60) (width 0.25) (layer "F.Cu") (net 1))
 (segment (start 122.614511 63.674511) (end 121.54 62.6) (width 0.25) (layer "F.Cu") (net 2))
 (segment (start 143.7 63.8) (end 143.675 63.8) (width 0.127) (layer "F.Cu") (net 2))
 (segment (start 140.375 60.5) (end 143.675 63.8) (width 0.25) (layer "F.Cu") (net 2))
 (segment (start 129.84 62.5) (end 131.84 60.5) (width 0.25) (layer "F.Cu") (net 2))
 (segment (start 143.8 63.925) (end 143.8 63.9) (width 0.127) (layer "F.Cu") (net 2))
 (segment (start 131.84 60.5) (end 140.375 60.5) (width 0.25) (layer "F.Cu") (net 2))
 (segment (start 132.1 60.5) (end 131.9 60.5) (width 0.127) (layer "F.Cu") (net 2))
 (segment (start 131.84 60.5) (end 132.1 60.5) (width 0.25) (layer "F.Cu") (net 2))
 (segment (start 144.935 65.06) (end 143.8 63.925) (width 0.127) (layer "F.Cu") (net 2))
 (segment (start 144.935 75.79) (end 144.935 65.06) (width 0.127) (layer "F.Cu") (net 2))
 (segment (start 128.765489 63.674511) (end 122.614511 63.674511) (width 0.25) (layer "F.Cu") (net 2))
 (segment (start 143.8 63.9) (end 143.7 63.8) (width 0.127) (layer "F.Cu") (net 2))
 (segment (start 129.84 62.6) (end 128.765489 63.674511) (width 0.25) (layer "F.Cu") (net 2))
 (segment (start 157 67.6) (end 157 73.25) (width 0.127) (layer "F.Cu") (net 6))
 (segment (start 155.73 73.25) (end 155.73 67.6) (width 0.127) (layer "F.Cu") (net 7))
 (segment (start 154.46 67.6) (end 154.46 73.25) (width 0.127) (layer "F.Cu") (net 8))
 (segment (start 153.19 73.25) (end 153.19 67.6) (width 0.127) (layer "F.Cu") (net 9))
 (segment (start 151.92 67.6) (end 151.92 73.25) (width 0.127) (layer "F.Cu") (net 10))
 (segment (start 150.65 67.6) (end 150.65 73.25) (width 0.127) (layer "F.Cu") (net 11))
 (segment (start 149.38 73.25) (end 149.38 67.6) (width 0.127) (layer "F.Cu") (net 12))
 (segment (start 148.11 67.6) (end 148.11 73.25) (width 0.127) (layer "F.Cu") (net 13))
 (segment (start 144.3 67.6) (end 144.3 73.25) (width 0.127) (layer "F.Cu") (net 14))
 (segment (start 143.03 67.6) (end 143.03 73.25) (width 0.127) (layer "F.Cu") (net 15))
 (segment (start 141.76 67.6) (end 141.76 73.25) (width 0.127) (layer "F.Cu") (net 16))
 (segment (start 156.365 65.06) (end 156.365 75.79) (width 0.127) (layer "F.Cu") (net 17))
 (segment (start 155.095 75.79) (end 155.095 65.06) (width 0.127) (layer "F.Cu") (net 18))
 (segment (start 153.825 65.06) (end 153.825 75.79) (width 0.127) (layer "F.Cu") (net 19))
 (segment (start 152.555 75.79) (end 152.555 65.06) (width 0.127) (layer "F.Cu") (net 20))
 (segment (start 151.285 65.06) (end 151.285 75.79) (width 0.127) (layer "F.Cu") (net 21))
 (segment (start 150.015 75.79) (end 150.015 65.06) (width 0.127) (layer "F.Cu") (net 22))
 (segment (start 148.745 65.06) (end 148.745 75.79) (width 0.127) (layer "F.Cu") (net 23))
 (segment (start 147.475 75.79) (end 147.475 65.06) (width 0.127) (layer "F.Cu") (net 24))
 (segment (start 143.665 65.06) (end 143.665 75.79) (width 0.127) (layer "F.Cu") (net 25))
 (segment (start 142.395 75.79) (end 142.395 65.06) (width 0.127) (layer "F.Cu") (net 26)))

